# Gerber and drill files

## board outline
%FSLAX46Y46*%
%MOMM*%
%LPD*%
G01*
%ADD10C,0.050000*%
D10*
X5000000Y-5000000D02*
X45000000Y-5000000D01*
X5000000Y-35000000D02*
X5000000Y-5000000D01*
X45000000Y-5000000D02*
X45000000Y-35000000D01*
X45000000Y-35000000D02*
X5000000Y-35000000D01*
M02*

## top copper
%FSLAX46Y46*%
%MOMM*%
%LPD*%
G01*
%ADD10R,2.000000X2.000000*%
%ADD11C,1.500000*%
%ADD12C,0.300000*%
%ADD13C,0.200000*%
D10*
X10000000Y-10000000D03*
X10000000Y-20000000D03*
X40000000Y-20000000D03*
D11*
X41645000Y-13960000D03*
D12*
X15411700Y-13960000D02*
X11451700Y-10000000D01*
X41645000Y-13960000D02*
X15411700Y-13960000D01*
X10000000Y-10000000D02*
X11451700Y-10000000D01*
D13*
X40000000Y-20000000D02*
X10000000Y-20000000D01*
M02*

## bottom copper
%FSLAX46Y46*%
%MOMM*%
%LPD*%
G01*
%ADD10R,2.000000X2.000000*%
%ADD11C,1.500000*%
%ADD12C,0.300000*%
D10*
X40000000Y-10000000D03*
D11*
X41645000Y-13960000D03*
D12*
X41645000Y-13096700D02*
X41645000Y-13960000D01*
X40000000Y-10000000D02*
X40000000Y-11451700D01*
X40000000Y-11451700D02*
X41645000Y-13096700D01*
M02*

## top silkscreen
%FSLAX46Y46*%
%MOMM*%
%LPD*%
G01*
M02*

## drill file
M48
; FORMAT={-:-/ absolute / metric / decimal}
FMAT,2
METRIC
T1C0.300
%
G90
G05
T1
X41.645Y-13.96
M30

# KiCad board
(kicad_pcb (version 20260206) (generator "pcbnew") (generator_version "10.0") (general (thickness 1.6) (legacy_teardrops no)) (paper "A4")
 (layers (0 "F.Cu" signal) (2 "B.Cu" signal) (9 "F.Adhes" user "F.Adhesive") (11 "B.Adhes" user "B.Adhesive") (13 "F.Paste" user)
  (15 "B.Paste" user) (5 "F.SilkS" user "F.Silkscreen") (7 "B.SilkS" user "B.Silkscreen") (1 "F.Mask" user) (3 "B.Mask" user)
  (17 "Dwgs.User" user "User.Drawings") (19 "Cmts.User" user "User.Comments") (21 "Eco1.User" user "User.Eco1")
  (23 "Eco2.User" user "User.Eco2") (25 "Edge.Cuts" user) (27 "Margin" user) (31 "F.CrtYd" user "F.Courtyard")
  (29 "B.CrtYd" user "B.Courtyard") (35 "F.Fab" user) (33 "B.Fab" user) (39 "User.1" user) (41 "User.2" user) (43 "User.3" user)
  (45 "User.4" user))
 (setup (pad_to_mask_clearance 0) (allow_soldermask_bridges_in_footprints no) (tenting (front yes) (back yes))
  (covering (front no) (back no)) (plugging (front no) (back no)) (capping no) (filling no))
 (gr_line (start 5 5) (end 45 5) (stroke (width 0.05) (type default)) (layer "Edge.Cuts"))
 (gr_line (start 5 35) (end 5 5) (stroke (width 0.05) (type default)) (layer "Edge.Cuts"))
 (gr_line (start 45 5) (end 45 35) (stroke (width 0.05) (type default)) (layer "Edge.Cuts"))
 (gr_line (start 45 35) (end 5 35) (stroke (width 0.05) (type default)) (layer "Edge.Cuts"))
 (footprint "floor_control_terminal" (layer "F.Cu") (at 10 10)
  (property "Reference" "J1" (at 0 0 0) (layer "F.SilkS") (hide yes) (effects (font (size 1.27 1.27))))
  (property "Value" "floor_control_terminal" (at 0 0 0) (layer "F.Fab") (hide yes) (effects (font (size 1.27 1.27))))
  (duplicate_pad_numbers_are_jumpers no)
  (pad "1" smd rect (at 0 0) (size 2 2) (layers "F.Cu" "F.Paste" "F.Mask") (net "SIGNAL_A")))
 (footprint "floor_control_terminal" (layer "B.Cu") (at 40 10)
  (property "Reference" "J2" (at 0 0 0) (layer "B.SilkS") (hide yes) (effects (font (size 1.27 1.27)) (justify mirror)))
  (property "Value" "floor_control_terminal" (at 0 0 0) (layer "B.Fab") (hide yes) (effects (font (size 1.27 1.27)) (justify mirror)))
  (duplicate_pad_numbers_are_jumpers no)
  (pad "1" smd rect (at 0 0) (size 2 2) (layers "B.Cu" "B.Paste" "B.Mask") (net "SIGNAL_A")))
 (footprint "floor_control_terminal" (layer "F.Cu") (at 10 20)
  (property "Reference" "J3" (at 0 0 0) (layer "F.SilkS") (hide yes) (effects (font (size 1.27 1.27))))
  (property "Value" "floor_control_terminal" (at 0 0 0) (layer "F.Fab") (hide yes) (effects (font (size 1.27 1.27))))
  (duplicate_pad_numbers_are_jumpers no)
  (pad "1" smd rect (at 0 0) (size 2 2) (layers "F.Cu" "F.Paste" "F.Mask") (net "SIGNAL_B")))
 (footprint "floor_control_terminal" (layer "F.Cu") (at 40 20)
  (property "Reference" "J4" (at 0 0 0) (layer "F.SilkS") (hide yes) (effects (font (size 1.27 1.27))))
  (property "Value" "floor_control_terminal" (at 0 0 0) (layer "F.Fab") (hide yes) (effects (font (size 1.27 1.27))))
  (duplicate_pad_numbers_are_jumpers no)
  (pad "1" smd rect (at 0 0) (size 2 2) (layers "F.Cu" "F.Paste" "F.Mask") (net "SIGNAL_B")))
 (segment (start 15.4117 13.96) (end 11.4517 10) (width 0.3) (layer "F.Cu") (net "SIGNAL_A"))
 (segment (start 41.645 13.96) (end 15.4117 13.96) (width 0.3) (layer "F.Cu") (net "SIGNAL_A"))
 (segment (start 10 10) (end 11.4517 10) (width 0.3) (layer "F.Cu") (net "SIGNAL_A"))
 (via (at 41.645 13.96) (size 1.5) (drill 0.3) (layers "F.Cu" "B.Cu") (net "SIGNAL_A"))
 (segment (start 41.645 13.0967) (end 41.645 13.96) (width 0.3) (layer "B.Cu") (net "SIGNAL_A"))
 (segment (start 40 10) (end 40 11.4517) (width 0.3) (layer "B.Cu") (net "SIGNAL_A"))
 (segment (start 40 11.4517) (end 41.645 13.0967) (width 0.3) (layer "B.Cu") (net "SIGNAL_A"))
 (segment (start 40 20) (end 10 20) (width 0.2) (layer "F.Cu") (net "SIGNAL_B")))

